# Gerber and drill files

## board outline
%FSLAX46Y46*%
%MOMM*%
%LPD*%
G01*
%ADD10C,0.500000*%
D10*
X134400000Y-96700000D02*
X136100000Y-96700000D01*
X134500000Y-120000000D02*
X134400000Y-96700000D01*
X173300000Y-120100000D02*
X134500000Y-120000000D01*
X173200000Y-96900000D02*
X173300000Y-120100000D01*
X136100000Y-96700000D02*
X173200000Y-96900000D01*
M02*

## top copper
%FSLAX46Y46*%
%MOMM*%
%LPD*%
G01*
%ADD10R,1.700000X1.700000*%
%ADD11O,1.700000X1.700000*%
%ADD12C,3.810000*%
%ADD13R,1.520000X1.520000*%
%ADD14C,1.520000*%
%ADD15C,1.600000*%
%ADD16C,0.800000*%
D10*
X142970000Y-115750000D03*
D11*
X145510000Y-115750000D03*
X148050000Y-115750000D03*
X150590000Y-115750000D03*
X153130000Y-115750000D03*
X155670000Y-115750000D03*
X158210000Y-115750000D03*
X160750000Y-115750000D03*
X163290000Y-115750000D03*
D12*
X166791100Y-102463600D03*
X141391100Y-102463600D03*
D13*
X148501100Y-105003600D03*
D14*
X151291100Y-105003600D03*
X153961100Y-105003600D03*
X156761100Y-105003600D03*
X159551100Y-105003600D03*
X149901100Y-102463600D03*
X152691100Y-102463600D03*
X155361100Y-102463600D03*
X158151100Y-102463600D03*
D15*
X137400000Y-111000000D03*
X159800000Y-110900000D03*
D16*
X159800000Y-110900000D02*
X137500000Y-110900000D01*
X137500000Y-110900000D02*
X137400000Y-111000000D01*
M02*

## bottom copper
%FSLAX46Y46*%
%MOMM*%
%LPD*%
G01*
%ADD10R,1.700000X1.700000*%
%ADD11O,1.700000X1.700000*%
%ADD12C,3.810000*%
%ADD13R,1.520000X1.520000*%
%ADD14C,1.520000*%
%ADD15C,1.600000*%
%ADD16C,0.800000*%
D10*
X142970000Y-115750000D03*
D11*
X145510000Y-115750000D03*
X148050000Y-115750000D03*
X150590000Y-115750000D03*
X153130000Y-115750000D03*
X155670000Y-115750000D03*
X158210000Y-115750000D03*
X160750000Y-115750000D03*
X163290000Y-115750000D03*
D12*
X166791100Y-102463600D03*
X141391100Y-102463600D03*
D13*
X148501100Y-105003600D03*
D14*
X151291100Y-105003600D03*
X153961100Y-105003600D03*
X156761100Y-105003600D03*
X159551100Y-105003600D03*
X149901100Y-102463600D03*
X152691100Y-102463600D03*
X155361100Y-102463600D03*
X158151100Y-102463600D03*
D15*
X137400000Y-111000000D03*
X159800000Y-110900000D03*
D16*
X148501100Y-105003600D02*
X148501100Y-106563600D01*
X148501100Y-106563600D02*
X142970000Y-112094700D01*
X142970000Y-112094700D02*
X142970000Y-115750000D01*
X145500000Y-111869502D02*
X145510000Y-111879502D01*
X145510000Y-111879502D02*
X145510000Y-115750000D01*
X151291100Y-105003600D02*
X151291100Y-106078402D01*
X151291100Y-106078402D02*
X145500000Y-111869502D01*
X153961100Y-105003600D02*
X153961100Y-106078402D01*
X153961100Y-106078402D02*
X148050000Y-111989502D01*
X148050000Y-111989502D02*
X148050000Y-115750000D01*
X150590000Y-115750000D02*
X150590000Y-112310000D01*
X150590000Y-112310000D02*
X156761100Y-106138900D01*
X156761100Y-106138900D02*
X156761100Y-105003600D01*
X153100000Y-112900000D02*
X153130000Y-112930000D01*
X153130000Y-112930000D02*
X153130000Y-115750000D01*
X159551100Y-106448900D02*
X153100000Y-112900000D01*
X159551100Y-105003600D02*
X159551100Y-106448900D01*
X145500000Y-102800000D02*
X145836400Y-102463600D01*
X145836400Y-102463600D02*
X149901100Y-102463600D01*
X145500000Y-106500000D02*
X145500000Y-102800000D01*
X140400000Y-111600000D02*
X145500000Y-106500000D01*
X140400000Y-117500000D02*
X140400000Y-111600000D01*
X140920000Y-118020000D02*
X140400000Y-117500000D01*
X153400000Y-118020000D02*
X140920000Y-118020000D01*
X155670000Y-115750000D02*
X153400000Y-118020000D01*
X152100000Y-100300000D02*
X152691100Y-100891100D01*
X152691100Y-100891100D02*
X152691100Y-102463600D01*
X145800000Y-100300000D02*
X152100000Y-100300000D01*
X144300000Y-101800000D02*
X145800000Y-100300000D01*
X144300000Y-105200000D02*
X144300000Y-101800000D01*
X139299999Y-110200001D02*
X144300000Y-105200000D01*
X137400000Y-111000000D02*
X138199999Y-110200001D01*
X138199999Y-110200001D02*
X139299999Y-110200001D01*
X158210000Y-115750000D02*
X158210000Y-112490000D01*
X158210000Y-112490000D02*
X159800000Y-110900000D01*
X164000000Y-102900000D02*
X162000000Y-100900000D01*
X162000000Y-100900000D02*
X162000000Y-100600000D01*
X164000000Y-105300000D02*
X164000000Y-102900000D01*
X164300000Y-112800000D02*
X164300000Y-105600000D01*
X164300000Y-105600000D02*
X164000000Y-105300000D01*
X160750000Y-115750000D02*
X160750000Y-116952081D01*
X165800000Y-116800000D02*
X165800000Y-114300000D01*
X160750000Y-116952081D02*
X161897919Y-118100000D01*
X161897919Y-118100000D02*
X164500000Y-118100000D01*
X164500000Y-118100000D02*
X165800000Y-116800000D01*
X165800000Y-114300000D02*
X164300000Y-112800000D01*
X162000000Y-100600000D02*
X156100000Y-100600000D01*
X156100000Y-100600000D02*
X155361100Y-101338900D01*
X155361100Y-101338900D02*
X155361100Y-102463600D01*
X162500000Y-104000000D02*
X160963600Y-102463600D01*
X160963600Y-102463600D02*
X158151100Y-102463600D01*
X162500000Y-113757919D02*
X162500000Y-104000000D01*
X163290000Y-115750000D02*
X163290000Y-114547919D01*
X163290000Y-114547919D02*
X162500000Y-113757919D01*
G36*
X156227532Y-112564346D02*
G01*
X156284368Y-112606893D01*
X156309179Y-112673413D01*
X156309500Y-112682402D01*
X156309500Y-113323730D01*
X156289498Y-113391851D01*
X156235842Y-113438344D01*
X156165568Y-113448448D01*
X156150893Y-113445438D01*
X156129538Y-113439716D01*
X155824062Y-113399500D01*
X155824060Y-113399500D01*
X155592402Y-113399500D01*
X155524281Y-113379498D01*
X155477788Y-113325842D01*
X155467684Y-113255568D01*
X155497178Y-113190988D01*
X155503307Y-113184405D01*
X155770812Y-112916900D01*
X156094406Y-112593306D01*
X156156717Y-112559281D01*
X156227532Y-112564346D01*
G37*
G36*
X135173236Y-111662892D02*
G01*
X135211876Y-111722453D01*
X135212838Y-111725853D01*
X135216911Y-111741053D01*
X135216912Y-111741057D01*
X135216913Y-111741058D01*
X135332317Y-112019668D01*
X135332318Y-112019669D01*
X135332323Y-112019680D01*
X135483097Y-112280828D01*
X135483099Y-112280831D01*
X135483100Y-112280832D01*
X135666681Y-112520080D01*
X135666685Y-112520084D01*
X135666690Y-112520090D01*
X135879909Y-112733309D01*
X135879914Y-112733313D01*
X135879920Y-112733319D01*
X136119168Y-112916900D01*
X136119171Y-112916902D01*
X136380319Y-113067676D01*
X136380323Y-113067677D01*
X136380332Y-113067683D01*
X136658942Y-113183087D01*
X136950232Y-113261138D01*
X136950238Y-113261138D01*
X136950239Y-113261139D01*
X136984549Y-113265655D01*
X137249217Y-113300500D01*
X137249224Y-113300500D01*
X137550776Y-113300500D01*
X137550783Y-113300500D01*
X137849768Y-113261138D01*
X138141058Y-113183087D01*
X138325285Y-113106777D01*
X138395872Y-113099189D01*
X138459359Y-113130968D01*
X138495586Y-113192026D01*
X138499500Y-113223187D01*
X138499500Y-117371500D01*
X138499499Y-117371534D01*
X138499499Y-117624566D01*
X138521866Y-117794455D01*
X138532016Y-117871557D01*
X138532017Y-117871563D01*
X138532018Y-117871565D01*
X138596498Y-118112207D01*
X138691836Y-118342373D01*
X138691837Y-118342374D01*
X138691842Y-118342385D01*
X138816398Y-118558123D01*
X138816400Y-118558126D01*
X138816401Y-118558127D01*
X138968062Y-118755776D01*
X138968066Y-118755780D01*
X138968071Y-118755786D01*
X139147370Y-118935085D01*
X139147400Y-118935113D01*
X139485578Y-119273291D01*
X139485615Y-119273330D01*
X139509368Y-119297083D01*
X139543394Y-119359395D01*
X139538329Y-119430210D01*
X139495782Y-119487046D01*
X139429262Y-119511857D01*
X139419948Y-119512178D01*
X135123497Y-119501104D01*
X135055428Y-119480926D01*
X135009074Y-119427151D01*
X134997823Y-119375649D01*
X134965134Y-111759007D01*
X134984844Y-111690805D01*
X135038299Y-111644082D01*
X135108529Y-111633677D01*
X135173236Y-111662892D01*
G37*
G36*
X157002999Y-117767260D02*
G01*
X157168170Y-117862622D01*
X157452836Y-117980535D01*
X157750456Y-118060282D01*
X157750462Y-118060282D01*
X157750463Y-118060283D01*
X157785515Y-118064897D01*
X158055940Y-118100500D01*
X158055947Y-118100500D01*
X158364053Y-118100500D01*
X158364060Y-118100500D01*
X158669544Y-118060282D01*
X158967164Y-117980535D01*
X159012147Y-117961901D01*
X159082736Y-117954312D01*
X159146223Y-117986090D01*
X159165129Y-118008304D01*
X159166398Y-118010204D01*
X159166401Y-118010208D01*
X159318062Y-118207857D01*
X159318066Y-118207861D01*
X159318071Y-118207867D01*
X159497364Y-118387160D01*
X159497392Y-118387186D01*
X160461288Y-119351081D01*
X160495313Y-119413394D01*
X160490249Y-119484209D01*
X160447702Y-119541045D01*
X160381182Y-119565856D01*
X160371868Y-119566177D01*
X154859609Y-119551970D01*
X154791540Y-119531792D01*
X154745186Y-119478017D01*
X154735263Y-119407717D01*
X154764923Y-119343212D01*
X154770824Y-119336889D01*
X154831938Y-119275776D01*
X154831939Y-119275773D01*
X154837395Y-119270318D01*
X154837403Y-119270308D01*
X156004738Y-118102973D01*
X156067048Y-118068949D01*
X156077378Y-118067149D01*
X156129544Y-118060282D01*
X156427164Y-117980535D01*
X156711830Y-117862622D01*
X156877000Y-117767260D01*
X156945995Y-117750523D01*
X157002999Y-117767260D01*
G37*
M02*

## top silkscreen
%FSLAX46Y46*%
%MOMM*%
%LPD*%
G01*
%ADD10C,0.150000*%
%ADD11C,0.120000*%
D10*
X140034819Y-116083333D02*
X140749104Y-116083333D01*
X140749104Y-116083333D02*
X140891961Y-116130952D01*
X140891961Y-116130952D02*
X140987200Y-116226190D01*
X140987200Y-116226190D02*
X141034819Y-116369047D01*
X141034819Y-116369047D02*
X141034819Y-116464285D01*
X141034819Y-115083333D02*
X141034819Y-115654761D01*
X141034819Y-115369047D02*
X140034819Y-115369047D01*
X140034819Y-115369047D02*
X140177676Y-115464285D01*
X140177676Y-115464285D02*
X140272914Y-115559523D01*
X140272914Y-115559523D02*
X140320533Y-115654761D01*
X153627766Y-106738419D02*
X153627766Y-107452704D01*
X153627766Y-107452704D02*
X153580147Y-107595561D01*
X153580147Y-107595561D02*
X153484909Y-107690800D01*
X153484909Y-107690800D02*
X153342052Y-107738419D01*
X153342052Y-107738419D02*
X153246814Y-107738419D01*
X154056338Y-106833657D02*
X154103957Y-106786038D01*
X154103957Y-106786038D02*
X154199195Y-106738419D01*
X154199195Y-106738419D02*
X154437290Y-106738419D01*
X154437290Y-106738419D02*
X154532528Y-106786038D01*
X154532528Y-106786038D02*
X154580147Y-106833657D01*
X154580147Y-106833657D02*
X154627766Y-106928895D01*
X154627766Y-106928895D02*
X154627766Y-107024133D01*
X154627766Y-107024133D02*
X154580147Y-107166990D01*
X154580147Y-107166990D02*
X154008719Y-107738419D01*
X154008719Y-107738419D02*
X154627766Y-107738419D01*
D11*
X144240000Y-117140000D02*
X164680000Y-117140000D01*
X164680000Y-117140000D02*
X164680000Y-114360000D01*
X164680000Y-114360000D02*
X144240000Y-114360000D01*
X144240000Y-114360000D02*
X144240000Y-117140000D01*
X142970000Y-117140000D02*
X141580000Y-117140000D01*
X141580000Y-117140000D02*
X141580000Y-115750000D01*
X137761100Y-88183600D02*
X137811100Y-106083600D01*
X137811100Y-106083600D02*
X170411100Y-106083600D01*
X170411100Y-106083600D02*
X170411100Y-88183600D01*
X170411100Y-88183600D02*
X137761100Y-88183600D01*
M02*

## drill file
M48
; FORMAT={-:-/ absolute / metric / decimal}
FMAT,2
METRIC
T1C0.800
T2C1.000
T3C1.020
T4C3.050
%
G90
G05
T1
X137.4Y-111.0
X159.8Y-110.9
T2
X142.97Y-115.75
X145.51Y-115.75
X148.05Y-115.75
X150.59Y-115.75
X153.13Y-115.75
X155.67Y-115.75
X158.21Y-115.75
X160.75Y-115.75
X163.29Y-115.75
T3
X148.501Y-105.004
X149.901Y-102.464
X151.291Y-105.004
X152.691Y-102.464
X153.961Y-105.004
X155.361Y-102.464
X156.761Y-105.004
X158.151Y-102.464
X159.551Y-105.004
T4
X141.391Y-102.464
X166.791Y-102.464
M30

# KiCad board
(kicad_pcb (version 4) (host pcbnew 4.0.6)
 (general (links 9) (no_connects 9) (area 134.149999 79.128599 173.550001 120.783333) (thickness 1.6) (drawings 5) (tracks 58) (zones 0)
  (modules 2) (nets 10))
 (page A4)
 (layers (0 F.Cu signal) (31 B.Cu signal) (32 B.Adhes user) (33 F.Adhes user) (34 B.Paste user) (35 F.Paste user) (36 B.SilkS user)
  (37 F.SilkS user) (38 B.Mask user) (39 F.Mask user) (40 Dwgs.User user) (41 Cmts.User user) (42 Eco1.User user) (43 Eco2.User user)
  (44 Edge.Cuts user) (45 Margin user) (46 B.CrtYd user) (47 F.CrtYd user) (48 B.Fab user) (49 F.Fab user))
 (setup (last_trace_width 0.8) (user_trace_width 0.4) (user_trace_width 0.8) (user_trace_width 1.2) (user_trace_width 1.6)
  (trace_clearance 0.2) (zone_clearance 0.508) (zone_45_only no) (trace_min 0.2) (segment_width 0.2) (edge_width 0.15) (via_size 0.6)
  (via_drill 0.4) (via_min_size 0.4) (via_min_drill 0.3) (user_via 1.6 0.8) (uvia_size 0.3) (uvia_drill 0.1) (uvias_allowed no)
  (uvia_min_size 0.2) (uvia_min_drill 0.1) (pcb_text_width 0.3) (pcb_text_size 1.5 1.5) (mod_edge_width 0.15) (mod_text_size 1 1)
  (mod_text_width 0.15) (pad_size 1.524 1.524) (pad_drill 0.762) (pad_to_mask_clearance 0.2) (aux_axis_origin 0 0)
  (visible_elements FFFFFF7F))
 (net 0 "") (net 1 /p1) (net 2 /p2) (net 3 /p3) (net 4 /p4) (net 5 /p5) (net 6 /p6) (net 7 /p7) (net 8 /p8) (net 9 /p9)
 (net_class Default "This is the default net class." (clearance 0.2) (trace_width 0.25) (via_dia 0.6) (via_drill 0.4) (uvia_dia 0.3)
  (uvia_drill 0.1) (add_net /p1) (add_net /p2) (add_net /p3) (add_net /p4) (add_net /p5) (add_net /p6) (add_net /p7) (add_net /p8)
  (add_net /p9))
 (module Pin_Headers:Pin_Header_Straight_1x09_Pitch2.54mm (layer F.Cu) (at 142.97 115.75 90)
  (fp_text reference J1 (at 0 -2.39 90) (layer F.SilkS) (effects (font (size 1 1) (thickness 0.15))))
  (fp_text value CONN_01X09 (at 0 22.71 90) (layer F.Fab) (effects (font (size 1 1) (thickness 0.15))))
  (fp_line (start -1.39 1.27) (end -1.39 21.71) (layer F.SilkS) (width 0.12))
  (fp_line (start -1.39 21.71) (end 1.39 21.71) (layer F.SilkS) (width 0.12))
  (fp_line (start 1.39 21.71) (end 1.39 1.27) (layer F.SilkS) (width 0.12))
  (fp_line (start 1.39 1.27) (end -1.39 1.27) (layer F.SilkS) (width 0.12))
  (fp_line (start -1.39 0) (end -1.39 -1.39) (layer F.SilkS) (width 0.12))
  (fp_line (start -1.39 -1.39) (end 0 -1.39) (layer F.SilkS) (width 0.12))
  (pad 1 thru_hole rect (at 0 0 90) (size 1.7 1.7) (drill 1) (layers *.Cu *.Mask) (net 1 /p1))
  (pad 2 thru_hole oval (at 0 2.54 90) (size 1.7 1.7) (drill 1) (layers *.Cu *.Mask) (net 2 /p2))
  (pad 3 thru_hole oval (at 0 5.08 90) (size 1.7 1.7) (drill 1) (layers *.Cu *.Mask) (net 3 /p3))
  (pad 4 thru_hole oval (at 0 7.62 90) (size 1.7 1.7) (drill 1) (layers *.Cu *.Mask) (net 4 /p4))
  (pad 5 thru_hole oval (at 0 10.16 90) (size 1.7 1.7) (drill 1) (layers *.Cu *.Mask) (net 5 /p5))
  (pad 6 thru_hole oval (at 0 12.7 90) (size 1.7 1.7) (drill 1) (layers *.Cu *.Mask) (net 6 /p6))
  (pad 7 thru_hole oval (at 0 15.24 90) (size 1.7 1.7) (drill 1) (layers *.Cu *.Mask) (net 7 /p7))
  (pad 8 thru_hole oval (at 0 17.78 90) (size 1.7 1.7) (drill 1) (layers *.Cu *.Mask) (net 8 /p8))
  (pad 9 thru_hole oval (at 0 20.32 90) (size 1.7 1.7) (drill 1) (layers *.Cu *.Mask) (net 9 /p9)))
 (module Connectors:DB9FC (layer F.Cu) (at 148.5011 105.0036)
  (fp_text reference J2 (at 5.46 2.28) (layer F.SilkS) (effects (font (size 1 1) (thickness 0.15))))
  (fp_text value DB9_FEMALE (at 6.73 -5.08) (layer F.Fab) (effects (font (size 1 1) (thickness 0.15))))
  (fp_line (start -10.74 -16.82) (end -10.69 1.08) (layer F.SilkS) (width 0.12))
  (fp_line (start -10.69 1.08) (end 21.91 1.08) (layer F.SilkS) (width 0.12))
  (fp_line (start 21.91 1.08) (end 21.91 -16.82) (layer F.SilkS) (width 0.12))
  (fp_line (start 21.91 -16.82) (end -10.74 -16.82) (layer F.SilkS) (width 0.12))
  (pad "" thru_hole circle (at 18.29 -2.54) (size 3.81 3.81) (drill 3.05) (layers *.Cu *.Mask))
  (pad "" thru_hole circle (at -7.11 -2.54) (size 3.81 3.81) (drill 3.05) (layers *.Cu *.Mask))
  (pad 1 thru_hole rect (at 0 0) (size 1.52 1.52) (drill 1.02) (layers *.Cu *.Mask) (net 1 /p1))
  (pad 2 thru_hole circle (at 2.79 0) (size 1.52 1.52) (drill 1.02) (layers *.Cu *.Mask) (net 2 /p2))
  (pad 3 thru_hole circle (at 5.46 0) (size 1.52 1.52) (drill 1.02) (layers *.Cu *.Mask) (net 3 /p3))
  (pad 4 thru_hole circle (at 8.26 0) (size 1.52 1.52) (drill 1.02) (layers *.Cu *.Mask) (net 4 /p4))
  (pad 5 thru_hole circle (at 11.05 0) (size 1.52 1.52) (drill 1.02) (layers *.Cu *.Mask) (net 5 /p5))
  (pad 6 thru_hole circle (at 1.4 -2.54) (size 1.52 1.52) (drill 1.02) (layers *.Cu *.Mask) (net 6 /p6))
  (pad 7 thru_hole circle (at 4.19 -2.54) (size 1.52 1.52) (drill 1.02) (layers *.Cu *.Mask) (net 7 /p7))
  (pad 8 thru_hole circle (at 6.86 -2.54) (size 1.52 1.52) (drill 1.02) (layers *.Cu *.Mask) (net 8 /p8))
  (pad 9 thru_hole circle (at 9.65 -2.54) (size 1.52 1.52) (drill 1.02) (layers *.Cu *.Mask) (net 9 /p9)))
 (gr_line (start 134.4 96.7) (end 136.1 96.7) (layer Edge.Cuts) (width 0.5))
 (gr_line (start 134.5 120) (end 134.4 96.7) (layer Edge.Cuts) (width 0.5))
 (gr_line (start 173.3 120.1) (end 134.5 120) (layer Edge.Cuts) (width 0.5))
 (gr_line (start 173.2 96.9) (end 173.3 120.1) (layer Edge.Cuts) (width 0.5))
 (gr_line (start 136.1 96.7) (end 173.2 96.9) (layer Edge.Cuts) (width 0.5))
 (segment (start 148.5011 105.0036) (end 148.5011 106.5636) (width 0.8) (layer B.Cu) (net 1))
 (segment (start 148.5011 106.5636) (end 142.97 112.0947) (width 0.8) (layer B.Cu) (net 1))
 (segment (start 142.97 112.0947) (end 142.97 115.75) (width 0.8) (layer B.Cu) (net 1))
 (segment (start 145.5 111.869502) (end 145.51 111.879502) (width 0.8) (layer B.Cu) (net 2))
 (segment (start 145.51 111.879502) (end 145.51 115.75) (width 0.8) (layer B.Cu) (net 2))
 (segment (start 151.2911 105.0036) (end 151.2911 106.078402) (width 0.8) (layer B.Cu) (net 2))
 (segment (start 151.2911 106.078402) (end 145.5 111.869502) (width 0.8) (layer B.Cu) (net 2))
 (segment (start 153.9611 105.0036) (end 153.9611 106.078402) (width 0.8) (layer B.Cu) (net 3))
 (segment (start 153.9611 106.078402) (end 148.05 111.989502) (width 0.8) (layer B.Cu) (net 3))
 (segment (start 148.05 111.989502) (end 148.05 115.75) (width 0.8) (layer B.Cu) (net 3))
 (segment (start 150.59 115.75) (end 150.59 112.31) (width 0.8) (layer B.Cu) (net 4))
 (segment (start 150.59 112.31) (end 156.7611 106.1389) (width 0.8) (layer B.Cu) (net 4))
 (segment (start 156.7611 106.1389) (end 156.7611 105.0036) (width 0.8) (layer B.Cu) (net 4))
 (segment (start 153.1 112.9) (end 153.13 112.93) (width 0.8) (layer B.Cu) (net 5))
 (segment (start 153.13 112.93) (end 153.13 115.75) (width 0.8) (layer B.Cu) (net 5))
 (segment (start 159.5511 106.4489) (end 153.1 112.9) (width 0.8) (layer B.Cu) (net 5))
 (segment (start 159.5511 105.0036) (end 159.5511 106.4489) (width 0.8) (layer B.Cu) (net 5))
 (segment (start 145.5 102.8) (end 145.8364 102.4636) (width 0.8) (layer B.Cu) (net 6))
 (segment (start 145.8364 102.4636) (end 149.9011 102.4636) (width 0.8) (layer B.Cu) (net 6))
 (segment (start 145.5 106.5) (end 145.5 102.8) (width 0.8) (layer B.Cu) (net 6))
 (segment (start 140.4 111.6) (end 145.5 106.5) (width 0.8) (layer B.Cu) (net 6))
 (segment (start 140.4 117.5) (end 140.4 111.6) (width 0.8) (layer B.Cu) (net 6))
 (segment (start 140.92 118.02) (end 140.4 117.5) (width 0.8) (layer B.Cu) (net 6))
 (segment (start 153.4 118.02) (end 140.92 118.02) (width 0.8) (layer B.Cu) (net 6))
 (segment (start 155.67 115.75) (end 153.4 118.02) (width 0.8) (layer B.Cu) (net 6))
 (segment (start 152.1 100.3) (end 152.6911 100.8911) (width 0.8) (layer B.Cu) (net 7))
 (segment (start 152.6911 100.8911) (end 152.6911 102.4636) (width 0.8) (layer B.Cu) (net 7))
 (segment (start 145.8 100.3) (end 152.1 100.3) (width 0.8) (layer B.Cu) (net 7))
 (segment (start 144.3 101.8) (end 145.8 100.3) (width 0.8) (layer B.Cu) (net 7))
 (segment (start 144.3 105.2) (end 144.3 101.8) (width 0.8) (layer B.Cu) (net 7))
 (segment (start 139.299999 110.200001) (end 144.3 105.2) (width 0.8) (layer B.Cu) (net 7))
 (segment (start 137.4 111) (end 138.199999 110.200001) (width 0.8) (layer B.Cu) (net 7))
 (segment (start 138.199999 110.200001) (end 139.299999 110.200001) (width 0.8) (layer B.Cu) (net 7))
 (segment (start 159.8 110.9) (end 137.5 110.9) (width 0.8) (layer F.Cu) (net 7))
 (via (at 137.4 111) (size 1.6) (drill 0.8) (layers F.Cu B.Cu) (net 7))
 (segment (start 137.5 110.9) (end 137.4 111) (width 0.8) (layer F.Cu) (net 7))
 (segment (start 158.21 115.75) (end 158.21 112.49) (width 0.8) (layer B.Cu) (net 7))
 (segment (start 158.21 112.49) (end 159.8 110.9) (width 0.8) (layer B.Cu) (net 7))
 (via (at 159.8 110.9) (size 1.6) (drill 0.8) (layers F.Cu B.Cu) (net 7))
 (segment (start 164 102.9) (end 162 100.9) (width 0.8) (layer B.Cu) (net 8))
 (segment (start 162 100.9) (end 162 100.6) (width 0.8) (layer B.Cu) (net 8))
 (segment (start 164 105.3) (end 164 102.9) (width 0.8) (layer B.Cu) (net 8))
 (segment (start 164.3 112.8) (end 164.3 105.6) (width 0.8) (layer B.Cu) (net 8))
 (segment (start 164.3 105.6) (end 164 105.3) (width 0.8) (layer B.Cu) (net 8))
 (segment (start 160.75 115.75) (end 160.75 116.952081) (width 0.8) (layer B.Cu) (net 8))
 (segment (start 165.8 116.8) (end 165.8 114.3) (width 0.8) (layer B.Cu) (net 8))
 (segment (start 160.75 116.952081) (end 161.897919 118.1) (width 0.8) (layer B.Cu) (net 8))
 (segment (start 161.897919 118.1) (end 164.5 118.1) (width 0.8) (layer B.Cu) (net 8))
 (segment (start 164.5 118.1) (end 165.8 116.8) (width 0.8) (layer B.Cu) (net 8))
 (segment (start 165.8 114.3) (end 164.3 112.8) (width 0.8) (layer B.Cu) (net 8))
 (segment (start 162 100.6) (end 156.1 100.6) (width 0.8) (layer B.Cu) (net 8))
 (segment (start 156.1 100.6) (end 155.3611 101.3389) (width 0.8) (layer B.Cu) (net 8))
 (segment (start 155.3611 101.3389) (end 155.3611 102.4636) (width 0.8) (layer B.Cu) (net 8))
 (segment (start 162.5 104) (end 160.9636 102.4636) (width 0.8) (layer B.Cu) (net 9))
 (segment (start 160.9636 102.4636) (end 158.1511 102.4636) (width 0.8) (layer B.Cu) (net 9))
 (segment (start 162.5 113.757919) (end 162.5 104) (width 0.8) (layer B.Cu) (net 9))
 (segment (start 163.29 115.75) (end 163.29 114.547919) (width 0.8) (layer B.Cu) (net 9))
 (segment (start 163.29 114.547919) (end 162.5 113.757919) (width 0.8) (layer B.Cu) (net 9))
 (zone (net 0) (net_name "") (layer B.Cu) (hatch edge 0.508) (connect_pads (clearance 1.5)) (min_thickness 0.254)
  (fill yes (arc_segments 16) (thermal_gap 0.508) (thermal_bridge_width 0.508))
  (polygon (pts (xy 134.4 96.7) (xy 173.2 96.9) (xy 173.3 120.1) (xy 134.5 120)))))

